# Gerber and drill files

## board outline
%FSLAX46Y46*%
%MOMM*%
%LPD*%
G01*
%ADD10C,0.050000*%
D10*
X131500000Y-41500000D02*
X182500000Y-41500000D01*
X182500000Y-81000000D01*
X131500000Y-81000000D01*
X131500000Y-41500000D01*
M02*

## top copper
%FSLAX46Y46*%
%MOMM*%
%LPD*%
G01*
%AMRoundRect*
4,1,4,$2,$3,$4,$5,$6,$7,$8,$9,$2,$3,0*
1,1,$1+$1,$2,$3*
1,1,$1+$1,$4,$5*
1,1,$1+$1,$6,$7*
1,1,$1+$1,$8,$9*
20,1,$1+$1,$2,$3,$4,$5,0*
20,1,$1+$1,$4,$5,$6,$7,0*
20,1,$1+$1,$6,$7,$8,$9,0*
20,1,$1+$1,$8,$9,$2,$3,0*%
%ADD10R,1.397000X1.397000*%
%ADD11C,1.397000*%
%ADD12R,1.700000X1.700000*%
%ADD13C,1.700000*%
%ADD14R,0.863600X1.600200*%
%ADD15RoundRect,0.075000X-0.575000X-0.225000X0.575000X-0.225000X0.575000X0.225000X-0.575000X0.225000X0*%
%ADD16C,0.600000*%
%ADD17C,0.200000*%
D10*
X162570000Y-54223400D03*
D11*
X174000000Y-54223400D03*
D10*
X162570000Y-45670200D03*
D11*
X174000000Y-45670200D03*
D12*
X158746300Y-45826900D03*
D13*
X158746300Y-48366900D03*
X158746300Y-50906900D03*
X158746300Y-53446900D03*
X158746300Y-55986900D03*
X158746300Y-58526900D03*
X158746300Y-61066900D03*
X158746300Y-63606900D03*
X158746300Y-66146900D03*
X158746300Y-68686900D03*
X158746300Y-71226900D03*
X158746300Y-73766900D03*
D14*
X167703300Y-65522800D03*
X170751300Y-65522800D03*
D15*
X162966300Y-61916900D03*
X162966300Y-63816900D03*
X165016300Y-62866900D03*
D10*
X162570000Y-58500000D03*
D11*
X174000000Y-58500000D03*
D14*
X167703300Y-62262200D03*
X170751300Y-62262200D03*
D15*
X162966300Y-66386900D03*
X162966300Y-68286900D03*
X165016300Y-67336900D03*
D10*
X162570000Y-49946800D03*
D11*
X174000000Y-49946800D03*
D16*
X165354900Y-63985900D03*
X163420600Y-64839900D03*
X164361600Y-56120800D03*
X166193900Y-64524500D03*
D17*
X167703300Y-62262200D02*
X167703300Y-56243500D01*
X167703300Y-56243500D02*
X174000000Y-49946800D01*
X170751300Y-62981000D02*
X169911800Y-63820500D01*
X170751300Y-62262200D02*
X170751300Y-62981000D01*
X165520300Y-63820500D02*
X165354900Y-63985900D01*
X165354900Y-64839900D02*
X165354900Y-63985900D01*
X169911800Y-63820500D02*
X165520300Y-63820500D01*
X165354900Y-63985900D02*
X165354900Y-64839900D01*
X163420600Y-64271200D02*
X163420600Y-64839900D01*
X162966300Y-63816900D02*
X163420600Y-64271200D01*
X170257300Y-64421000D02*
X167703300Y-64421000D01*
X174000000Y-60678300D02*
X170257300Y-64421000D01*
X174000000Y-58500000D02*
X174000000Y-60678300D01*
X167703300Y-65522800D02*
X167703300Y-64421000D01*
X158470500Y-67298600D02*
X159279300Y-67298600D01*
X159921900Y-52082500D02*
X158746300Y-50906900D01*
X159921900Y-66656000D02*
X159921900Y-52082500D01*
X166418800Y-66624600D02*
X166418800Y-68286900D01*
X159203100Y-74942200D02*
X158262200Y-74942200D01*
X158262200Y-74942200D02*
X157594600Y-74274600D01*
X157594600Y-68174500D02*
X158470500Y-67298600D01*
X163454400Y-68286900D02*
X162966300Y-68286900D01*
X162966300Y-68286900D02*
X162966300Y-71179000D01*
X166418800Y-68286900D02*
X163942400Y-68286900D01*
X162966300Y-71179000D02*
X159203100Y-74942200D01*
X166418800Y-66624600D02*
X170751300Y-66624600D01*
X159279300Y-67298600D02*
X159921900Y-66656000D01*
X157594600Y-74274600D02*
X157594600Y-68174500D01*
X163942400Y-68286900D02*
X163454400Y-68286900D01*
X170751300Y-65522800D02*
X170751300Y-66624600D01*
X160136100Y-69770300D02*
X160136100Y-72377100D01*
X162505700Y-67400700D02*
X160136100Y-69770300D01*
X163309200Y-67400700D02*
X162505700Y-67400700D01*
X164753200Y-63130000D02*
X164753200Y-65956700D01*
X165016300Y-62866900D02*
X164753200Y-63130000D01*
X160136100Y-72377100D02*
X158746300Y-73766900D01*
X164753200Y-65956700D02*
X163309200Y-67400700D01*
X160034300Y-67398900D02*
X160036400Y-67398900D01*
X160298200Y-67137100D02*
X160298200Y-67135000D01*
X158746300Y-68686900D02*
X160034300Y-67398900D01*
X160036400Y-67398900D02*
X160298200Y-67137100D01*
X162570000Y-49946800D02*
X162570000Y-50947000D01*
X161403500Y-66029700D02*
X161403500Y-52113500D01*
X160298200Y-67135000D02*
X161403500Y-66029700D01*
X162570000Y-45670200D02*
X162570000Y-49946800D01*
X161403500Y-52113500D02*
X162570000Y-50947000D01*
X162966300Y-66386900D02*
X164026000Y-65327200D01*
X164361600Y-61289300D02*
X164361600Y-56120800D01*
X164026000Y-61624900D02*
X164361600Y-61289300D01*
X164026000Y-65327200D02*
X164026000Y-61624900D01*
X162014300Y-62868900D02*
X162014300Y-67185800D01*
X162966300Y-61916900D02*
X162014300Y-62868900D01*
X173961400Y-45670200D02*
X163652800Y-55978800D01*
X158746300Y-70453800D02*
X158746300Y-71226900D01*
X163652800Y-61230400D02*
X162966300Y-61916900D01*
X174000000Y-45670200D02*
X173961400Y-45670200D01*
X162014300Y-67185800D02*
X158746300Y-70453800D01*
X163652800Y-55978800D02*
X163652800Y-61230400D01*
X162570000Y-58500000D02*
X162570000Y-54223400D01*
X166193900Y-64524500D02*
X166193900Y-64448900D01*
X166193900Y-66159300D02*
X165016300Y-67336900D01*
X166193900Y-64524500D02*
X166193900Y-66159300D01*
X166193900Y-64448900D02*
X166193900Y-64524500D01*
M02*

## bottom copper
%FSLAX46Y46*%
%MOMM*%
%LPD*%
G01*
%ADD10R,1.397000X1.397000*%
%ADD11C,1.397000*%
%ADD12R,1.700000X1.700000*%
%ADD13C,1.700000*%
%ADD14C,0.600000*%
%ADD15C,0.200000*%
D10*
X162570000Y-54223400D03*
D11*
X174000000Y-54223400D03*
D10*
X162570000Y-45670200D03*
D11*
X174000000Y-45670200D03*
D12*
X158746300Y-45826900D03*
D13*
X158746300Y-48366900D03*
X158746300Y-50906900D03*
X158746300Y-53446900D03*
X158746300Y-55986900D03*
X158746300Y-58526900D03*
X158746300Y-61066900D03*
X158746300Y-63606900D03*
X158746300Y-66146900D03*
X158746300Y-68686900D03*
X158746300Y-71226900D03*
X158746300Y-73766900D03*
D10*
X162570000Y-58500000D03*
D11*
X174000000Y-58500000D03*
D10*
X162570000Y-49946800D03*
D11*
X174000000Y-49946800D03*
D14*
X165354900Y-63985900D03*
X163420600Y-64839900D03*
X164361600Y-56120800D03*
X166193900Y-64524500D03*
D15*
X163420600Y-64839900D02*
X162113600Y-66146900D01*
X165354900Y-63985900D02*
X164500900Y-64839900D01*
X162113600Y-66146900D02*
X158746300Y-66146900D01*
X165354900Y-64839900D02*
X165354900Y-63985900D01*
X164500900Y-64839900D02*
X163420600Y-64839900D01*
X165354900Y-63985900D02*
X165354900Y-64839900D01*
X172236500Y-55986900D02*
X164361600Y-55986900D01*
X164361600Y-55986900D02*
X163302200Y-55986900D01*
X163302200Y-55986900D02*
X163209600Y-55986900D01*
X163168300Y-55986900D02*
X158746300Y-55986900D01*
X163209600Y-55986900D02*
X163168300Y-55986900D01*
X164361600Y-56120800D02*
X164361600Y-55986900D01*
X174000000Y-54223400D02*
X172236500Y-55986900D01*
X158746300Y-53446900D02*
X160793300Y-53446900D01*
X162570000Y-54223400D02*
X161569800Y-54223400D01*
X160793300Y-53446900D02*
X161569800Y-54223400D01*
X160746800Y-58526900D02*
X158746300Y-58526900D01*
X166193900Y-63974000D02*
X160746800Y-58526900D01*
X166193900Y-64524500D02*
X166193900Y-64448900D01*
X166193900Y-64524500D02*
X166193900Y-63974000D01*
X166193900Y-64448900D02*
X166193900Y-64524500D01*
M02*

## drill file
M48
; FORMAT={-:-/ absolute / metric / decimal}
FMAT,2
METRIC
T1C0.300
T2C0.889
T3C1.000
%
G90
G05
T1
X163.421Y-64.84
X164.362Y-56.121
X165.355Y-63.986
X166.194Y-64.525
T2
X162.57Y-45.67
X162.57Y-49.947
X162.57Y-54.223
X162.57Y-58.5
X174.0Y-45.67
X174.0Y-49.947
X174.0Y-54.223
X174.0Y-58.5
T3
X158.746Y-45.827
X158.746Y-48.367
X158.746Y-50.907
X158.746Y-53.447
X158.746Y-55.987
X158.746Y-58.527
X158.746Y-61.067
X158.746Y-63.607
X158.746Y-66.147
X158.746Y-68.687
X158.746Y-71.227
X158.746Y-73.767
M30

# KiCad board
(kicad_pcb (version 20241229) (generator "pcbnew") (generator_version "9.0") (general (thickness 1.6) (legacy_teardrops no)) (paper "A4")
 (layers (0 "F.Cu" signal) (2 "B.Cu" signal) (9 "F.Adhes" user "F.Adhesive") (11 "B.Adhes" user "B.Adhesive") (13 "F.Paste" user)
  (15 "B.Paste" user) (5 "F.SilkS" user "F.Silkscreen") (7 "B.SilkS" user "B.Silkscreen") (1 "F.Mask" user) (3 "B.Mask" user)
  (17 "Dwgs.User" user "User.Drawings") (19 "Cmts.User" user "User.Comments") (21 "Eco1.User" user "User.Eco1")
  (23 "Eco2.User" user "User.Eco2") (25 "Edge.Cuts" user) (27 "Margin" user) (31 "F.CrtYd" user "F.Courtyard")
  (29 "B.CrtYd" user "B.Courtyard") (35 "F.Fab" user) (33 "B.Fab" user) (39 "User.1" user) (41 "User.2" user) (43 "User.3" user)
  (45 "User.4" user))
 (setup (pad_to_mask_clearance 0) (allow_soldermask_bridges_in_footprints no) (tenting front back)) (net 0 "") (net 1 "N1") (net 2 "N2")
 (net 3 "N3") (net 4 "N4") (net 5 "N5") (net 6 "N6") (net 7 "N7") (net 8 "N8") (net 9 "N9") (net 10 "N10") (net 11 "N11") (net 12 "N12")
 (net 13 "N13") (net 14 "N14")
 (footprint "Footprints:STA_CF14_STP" (layer "F.Cu") (at 162.57 54.2234)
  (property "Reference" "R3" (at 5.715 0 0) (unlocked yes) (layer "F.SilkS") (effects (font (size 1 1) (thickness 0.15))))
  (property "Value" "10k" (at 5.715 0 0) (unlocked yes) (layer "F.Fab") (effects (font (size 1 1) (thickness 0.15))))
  (pad "1" thru_hole rect (at 0 0) (size 1.397 1.397) (drill 0.889) (layers "*.Cu" "*.Mask") (remove_unused_layers no) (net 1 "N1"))
  (pad "2" thru_hole circle (at 11.43 0) (size 1.397 1.397) (drill 0.889) (layers "*.Cu" "*.Mask") (remove_unused_layers no) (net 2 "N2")))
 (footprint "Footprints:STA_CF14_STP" (layer "F.Cu") (at 162.57 45.6702)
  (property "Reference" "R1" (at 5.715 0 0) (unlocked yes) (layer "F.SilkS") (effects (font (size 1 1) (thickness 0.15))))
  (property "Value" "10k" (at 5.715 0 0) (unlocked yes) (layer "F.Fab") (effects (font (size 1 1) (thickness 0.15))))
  (pad "1" thru_hole rect (at 0 0) (size 1.397 1.397) (drill 0.889) (layers "*.Cu" "*.Mask") (remove_unused_layers no) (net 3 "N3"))
  (pad "2" thru_hole circle (at 11.43 0) (size 1.397 1.397) (drill 0.889) (layers "*.Cu" "*.Mask") (remove_unused_layers no) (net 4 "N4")))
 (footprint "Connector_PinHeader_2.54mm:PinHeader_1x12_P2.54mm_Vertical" (layer "F.Cu") (at 158.7463 45.8269)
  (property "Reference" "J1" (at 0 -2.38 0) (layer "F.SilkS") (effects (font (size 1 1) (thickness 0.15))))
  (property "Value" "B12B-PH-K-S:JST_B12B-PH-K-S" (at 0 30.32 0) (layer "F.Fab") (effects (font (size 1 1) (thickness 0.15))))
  (pad "1" thru_hole rect (at 0 0) (size 1.7 1.7) (drill 1) (layers "*.Cu" "*.Mask") (remove_unused_layers no) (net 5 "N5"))
  (pad "2" thru_hole circle (at 0 2.54) (size 1.7 1.7) (drill 1) (layers "*.Cu" "*.Mask") (remove_unused_layers no) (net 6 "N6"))
  (pad "3" thru_hole circle (at 0 5.08) (size 1.7 1.7) (drill 1) (layers "*.Cu" "*.Mask") (remove_unused_layers no) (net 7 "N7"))
  (pad "4" thru_hole circle (at 0 7.62) (size 1.7 1.7) (drill 1) (layers "*.Cu" "*.Mask") (remove_unused_layers no) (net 1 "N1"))
  (pad "5" thru_hole circle (at 0 10.16) (size 1.7 1.7) (drill 1) (layers "*.Cu" "*.Mask") (remove_unused_layers no) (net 2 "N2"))
  (pad "6" thru_hole circle (at 0 12.7) (size 1.7 1.7) (drill 1) (layers "*.Cu" "*.Mask") (remove_unused_layers no) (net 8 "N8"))
  (pad "7" thru_hole circle (at 0 15.24) (size 1.7 1.7) (drill 1) (layers "*.Cu" "*.Mask") (remove_unused_layers no) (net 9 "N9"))
  (pad "8" thru_hole circle (at 0 17.78) (size 1.7 1.7) (drill 1) (layers "*.Cu" "*.Mask") (remove_unused_layers no) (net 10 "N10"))
  (pad "9" thru_hole circle (at 0 20.32) (size 1.7 1.7) (drill 1) (layers "*.Cu" "*.Mask") (remove_unused_layers no) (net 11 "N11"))
  (pad "10" thru_hole circle (at 0 22.86) (size 1.7 1.7) (drill 1) (layers "*.Cu" "*.Mask") (remove_unused_layers no) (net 3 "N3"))
  (pad "11" thru_hole circle (at 0 25.4) (size 1.7 1.7) (drill 1) (layers "*.Cu" "*.Mask") (remove_unused_layers no) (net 4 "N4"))
  (pad "12" thru_hole circle (at 0 27.94) (size 1.7 1.7) (drill 1) (layers "*.Cu" "*.Mask") (remove_unused_layers no) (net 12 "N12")))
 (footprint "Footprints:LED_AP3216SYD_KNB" (layer "F.Cu") (at 169.2273 65.5228)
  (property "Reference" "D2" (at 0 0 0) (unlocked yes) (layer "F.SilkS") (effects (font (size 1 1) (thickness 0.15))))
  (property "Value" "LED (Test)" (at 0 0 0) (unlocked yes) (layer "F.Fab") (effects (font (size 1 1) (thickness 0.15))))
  (pad "1" smd rect (at -1.524 0) (size 0.8636 1.6002) (layers "F.Cu" "F.Mask" "F.Paste") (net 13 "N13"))
  (pad "2" smd rect (at 1.524 0) (size 0.8636 1.6002) (layers "F.Cu" "F.Mask" "F.Paste") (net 7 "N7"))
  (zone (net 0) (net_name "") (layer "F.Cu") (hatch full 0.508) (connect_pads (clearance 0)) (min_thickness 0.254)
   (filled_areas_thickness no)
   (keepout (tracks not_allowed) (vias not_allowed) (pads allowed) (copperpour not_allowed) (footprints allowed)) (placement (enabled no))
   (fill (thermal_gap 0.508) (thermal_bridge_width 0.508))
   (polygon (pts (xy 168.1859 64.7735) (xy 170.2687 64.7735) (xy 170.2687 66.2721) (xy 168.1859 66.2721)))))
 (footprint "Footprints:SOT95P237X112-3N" (layer "F.Cu") (at 163.9913 62.8669)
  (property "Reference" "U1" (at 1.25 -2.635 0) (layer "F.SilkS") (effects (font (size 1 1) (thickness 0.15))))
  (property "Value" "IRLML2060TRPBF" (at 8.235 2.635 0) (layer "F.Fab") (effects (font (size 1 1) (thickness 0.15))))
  (pad "1" smd roundrect (at -1.025 -0.95) (size 1.3 0.6) (layers "F.Cu" "F.Mask" "F.Paste") (roundrect_rratio 0.125) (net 4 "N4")
   (solder_mask_margin 0.102))
  (pad "2" smd roundrect (at -1.025 0.95) (size 1.3 0.6) (layers "F.Cu" "F.Mask" "F.Paste") (roundrect_rratio 0.125) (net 11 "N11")
   (solder_mask_margin 0.102))
  (pad "3" smd roundrect (at 1.025 0) (size 1.3 0.6) (layers "F.Cu" "F.Mask" "F.Paste") (roundrect_rratio 0.125) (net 12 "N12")
   (solder_mask_margin 0.102)))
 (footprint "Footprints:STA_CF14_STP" (layer "F.Cu") (at 162.57 58.5)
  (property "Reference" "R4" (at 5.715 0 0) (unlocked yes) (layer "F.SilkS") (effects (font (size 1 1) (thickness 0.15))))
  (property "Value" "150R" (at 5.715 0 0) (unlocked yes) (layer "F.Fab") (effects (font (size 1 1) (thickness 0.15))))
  (pad "1" thru_hole rect (at 0 0) (size 1.397 1.397) (drill 0.889) (layers "*.Cu" "*.Mask") (remove_unused_layers no) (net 1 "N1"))
  (pad "2" thru_hole circle (at 11.43 0) (size 1.397 1.397) (drill 0.889) (layers "*.Cu" "*.Mask") (remove_unused_layers no) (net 13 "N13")))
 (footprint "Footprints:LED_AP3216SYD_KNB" (layer "F.Cu") (at 169.2273 62.2622)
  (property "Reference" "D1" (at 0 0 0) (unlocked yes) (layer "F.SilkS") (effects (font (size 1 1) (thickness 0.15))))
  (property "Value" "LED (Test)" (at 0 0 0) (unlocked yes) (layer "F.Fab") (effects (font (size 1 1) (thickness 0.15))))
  (pad "1" smd rect (at -1.524 0) (size 0.8636 1.6002) (layers "F.Cu" "F.Mask" "F.Paste") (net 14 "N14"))
  (pad "2" smd rect (at 1.524 0) (size 0.8636 1.6002) (layers "F.Cu" "F.Mask" "F.Paste") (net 11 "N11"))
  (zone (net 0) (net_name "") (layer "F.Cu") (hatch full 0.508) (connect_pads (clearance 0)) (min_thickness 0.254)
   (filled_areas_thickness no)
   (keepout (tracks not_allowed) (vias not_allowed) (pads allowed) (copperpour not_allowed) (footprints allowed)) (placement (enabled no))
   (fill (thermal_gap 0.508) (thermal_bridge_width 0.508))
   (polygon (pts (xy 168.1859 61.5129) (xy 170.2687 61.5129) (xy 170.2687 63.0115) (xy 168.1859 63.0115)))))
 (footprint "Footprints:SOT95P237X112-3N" (layer "F.Cu") (at 163.9913 67.3369)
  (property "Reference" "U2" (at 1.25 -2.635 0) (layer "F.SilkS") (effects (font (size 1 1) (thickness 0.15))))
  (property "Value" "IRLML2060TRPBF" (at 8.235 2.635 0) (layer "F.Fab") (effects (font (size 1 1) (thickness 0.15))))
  (pad "1" smd roundrect (at -1.025 -0.95) (size 1.3 0.6) (layers "F.Cu" "F.Mask" "F.Paste") (roundrect_rratio 0.125) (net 2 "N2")
   (solder_mask_margin 0.102))
  (pad "2" smd roundrect (at -1.025 0.95) (size 1.3 0.6) (layers "F.Cu" "F.Mask" "F.Paste") (roundrect_rratio 0.125) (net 7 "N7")
   (solder_mask_margin 0.102))
  (pad "3" smd roundrect (at 1.025 0) (size 1.3 0.6) (layers "F.Cu" "F.Mask" "F.Paste") (roundrect_rratio 0.125) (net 8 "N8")
   (solder_mask_margin 0.102)))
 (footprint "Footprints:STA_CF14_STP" (layer "F.Cu") (at 162.57 49.9468)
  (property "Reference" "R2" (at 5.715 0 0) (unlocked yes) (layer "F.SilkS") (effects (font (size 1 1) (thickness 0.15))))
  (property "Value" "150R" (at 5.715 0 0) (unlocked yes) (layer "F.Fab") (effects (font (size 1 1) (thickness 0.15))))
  (pad "1" thru_hole rect (at 0 0) (size 1.397 1.397) (drill 0.889) (layers "*.Cu" "*.Mask") (remove_unused_layers no) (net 3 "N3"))
  (pad "2" thru_hole circle (at 11.43 0) (size 1.397 1.397) (drill 0.889) (layers "*.Cu" "*.Mask") (remove_unused_layers no) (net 14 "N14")))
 (gr_rect (start 131.5 41.5) (end 182.5 81) (stroke (width 0.05) (type solid)) (fill no) (layer "Edge.Cuts"))
 (segment (start 167.7033 62.2622) (end 167.7033 56.2435) (width 0.2) (layer "F.Cu") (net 14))
 (segment (start 167.7033 56.2435) (end 174 49.9468) (width 0.2) (layer "F.Cu") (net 14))
 (segment (start 170.7513 62.981) (end 169.9118 63.8205) (width 0.2) (layer "F.Cu") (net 11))
 (segment (start 170.7513 62.2622) (end 170.7513 62.981) (width 0.2) (layer "F.Cu") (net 11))
 (segment (start 165.5203 63.8205) (end 165.3549 63.9859) (width 0.2) (layer "F.Cu") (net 11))
 (segment (start 165.3549 64.8399) (end 165.3549 63.9859) (width 0.2) (layer "F.Cu") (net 11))
 (segment (start 169.9118 63.8205) (end 165.5203 63.8205) (width 0.2) (layer "F.Cu") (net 11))
 (segment (start 165.3549 63.9859) (end 165.3549 64.8399) (width 0.2) (layer "F.Cu") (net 11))
 (segment (start 163.4206 64.2712) (end 163.4206 64.8399) (width 0.2) (layer "F.Cu") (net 11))
 (segment (start 162.9663 63.8169) (end 163.4206 64.2712) (width 0.2) (layer "F.Cu") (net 11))
 (via (at 165.3549 63.9859) (size 0.6) (drill 0.3) (layers "F.Cu" "B.Cu") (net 11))
 (via (at 163.4206 64.8399) (size 0.6) (drill 0.3) (layers "F.Cu" "B.Cu") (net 11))
 (segment (start 163.4206 64.8399) (end 162.1136 66.1469) (width 0.2) (layer "B.Cu") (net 11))
 (segment (start 165.3549 63.9859) (end 164.5009 64.8399) (width 0.2) (layer "B.Cu") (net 11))
 (segment (start 162.1136 66.1469) (end 158.7463 66.1469) (width 0.2) (layer "B.Cu") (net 11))
 (segment (start 165.3549 64.8399) (end 165.3549 63.9859) (width 0.2) (layer "B.Cu") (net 11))
 (segment (start 164.5009 64.8399) (end 163.4206 64.8399) (width 0.2) (layer "B.Cu") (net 11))
 (segment (start 165.3549 63.9859) (end 165.3549 64.8399) (width 0.2) (layer "B.Cu") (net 11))
 (segment (start 170.2573 64.421) (end 167.7033 64.421) (width 0.2) (layer "F.Cu") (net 13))
 (segment (start 174 60.6783) (end 170.2573 64.421) (width 0.2) (layer "F.Cu") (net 13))
 (segment (start 174 58.5) (end 174 60.6783) (width 0.2) (layer "F.Cu") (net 13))
 (segment (start 167.7033 65.5228) (end 167.7033 64.421) (width 0.2) (layer "F.Cu") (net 13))
 (segment (start 158.4705 67.2986) (end 159.2793 67.2986) (width 0.2) (layer "F.Cu") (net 7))
 (segment (start 159.9219 52.0825) (end 158.7463 50.9069) (width 0.2) (layer "F.Cu") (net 7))
 (segment (start 159.9219 66.656) (end 159.9219 52.0825) (width 0.2) (layer "F.Cu") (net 7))
 (segment (start 166.4188 66.6246) (end 166.4188 68.2869) (width 0.2) (layer "F.Cu") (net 7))
 (segment (start 159.2031 74.9422) (end 158.2622 74.9422) (width 0.2) (layer "F.Cu") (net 7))
 (segment (start 158.2622 74.9422) (end 157.5946 74.2746) (width 0.2) (layer "F.Cu") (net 7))
 (segment (start 157.5946 68.1745) (end 158.4705 67.2986) (width 0.2) (layer "F.Cu") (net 7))
 (segment (start 163.4544 68.2869) (end 162.9663 68.2869) (width 0.2) (layer "F.Cu") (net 7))
 (segment (start 162.9663 68.2869) (end 162.9663 71.179) (width 0.2) (layer "F.Cu") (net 7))
 (segment (start 166.4188 68.2869) (end 163.9424 68.2869) (width 0.2) (layer "F.Cu") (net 7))
 (segment (start 162.9663 71.179) (end 159.2031 74.9422) (width 0.2) (layer "F.Cu") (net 7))
 (segment (start 166.4188 66.6246) (end 170.7513 66.6246) (width 0.2) (layer "F.Cu") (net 7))
 (segment (start 159.2793 67.2986) (end 159.9219 66.656) (width 0.2) (layer "F.Cu") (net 7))
 (segment (start 157.5946 74.2746) (end 157.5946 68.1745) (width 0.2) (layer "F.Cu") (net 7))
 (segment (start 163.9424 68.2869) (end 163.4544 68.2869) (width 0.2) (layer "F.Cu") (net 7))
 (segment (start 170.7513 65.5228) (end 170.7513 66.6246) (width 0.2) (layer "F.Cu") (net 7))
 (segment (start 160.1361 69.7703) (end 160.1361 72.3771) (width 0.2) (layer "F.Cu") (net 12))
 (segment (start 162.5057 67.4007) (end 160.1361 69.7703) (width 0.2) (layer "F.Cu") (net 12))
 (segment (start 163.3092 67.4007) (end 162.5057 67.4007) (width 0.2) (layer "F.Cu") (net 12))
 (segment (start 164.7532 63.13) (end 164.7532 65.9567) (width 0.2) (layer "F.Cu") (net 12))
 (segment (start 165.0163 62.8669) (end 164.7532 63.13) (width 0.2) (layer "F.Cu") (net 12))
 (segment (start 160.1361 72.3771) (end 158.7463 73.7669) (width 0.2) (layer "F.Cu") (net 12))
 (segment (start 164.7532 65.9567) (end 163.3092 67.4007) (width 0.2) (layer "F.Cu") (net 12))
 (segment (start 160.0343 67.3989) (end 160.0364 67.3989) (width 0.2) (layer "F.Cu") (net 3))
 (segment (start 160.2982 67.1371) (end 160.2982 67.135) (width 0.2) (layer "F.Cu") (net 3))
 (segment (start 158.7463 68.6869) (end 160.0343 67.3989) (width 0.2) (layer "F.Cu") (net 3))
 (segment (start 160.0364 67.3989) (end 160.2982 67.1371) (width 0.2) (layer "F.Cu") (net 3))
 (segment (start 162.57 49.9468) (end 162.57 50.947) (width 0.2) (layer "F.Cu") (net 3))
 (segment (start 161.4035 66.0297) (end 161.4035 52.1135) (width 0.2) (layer "F.Cu") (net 3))
 (segment (start 160.2982 67.135) (end 161.4035 66.0297) (width 0.2) (layer "F.Cu") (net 3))
 (segment (start 162.57 45.6702) (end 162.57 49.9468) (width 0.2) (layer "F.Cu") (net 3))
 (segment (start 161.4035 52.1135) (end 162.57 50.947) (width 0.2) (layer "F.Cu") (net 3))
 (segment (start 162.9663 66.3869) (end 164.026 65.3272) (width 0.2) (layer "F.Cu") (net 2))
 (segment (start 164.3616 61.2893) (end 164.3616 56.1208) (width 0.2) (layer "F.Cu") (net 2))
 (segment (start 164.026 61.6249) (end 164.3616 61.2893) (width 0.2) (layer "F.Cu") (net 2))
 (segment (start 164.026 65.3272) (end 164.026 61.6249) (width 0.2) (layer "F.Cu") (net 2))
 (via (at 164.3616 56.1208) (size 0.6) (drill 0.3) (layers "F.Cu" "B.Cu") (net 2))
 (segment (start 172.2365 55.9869) (end 164.3616 55.9869) (width 0.2) (layer "B.Cu") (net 2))
 (segment (start 164.3616 55.9869) (end 163.3022 55.9869) (width 0.2) (layer "B.Cu") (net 2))
 (segment (start 163.3022 55.9869) (end 163.2096 55.9869) (width 0.2) (layer "B.Cu") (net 2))
 (segment (start 163.1683 55.9869) (end 158.7463 55.9869) (width 0.2) (layer "B.Cu") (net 2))
 (segment (start 163.2096 55.9869) (end 163.1683 55.9869) (width 0.2) (layer "B.Cu") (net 2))
 (segment (start 164.3616 56.1208) (end 164.3616 55.9869) (width 0.2) (layer "B.Cu") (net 2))
 (segment (start 174 54.2234) (end 172.2365 55.9869) (width 0.2) (layer "B.Cu") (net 2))
 (segment (start 162.0143 62.8689) (end 162.0143 67.1858) (width 0.2) (layer "F.Cu") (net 4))
 (segment (start 162.9663 61.9169) (end 162.0143 62.8689) (width 0.2) (layer "F.Cu") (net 4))
 (segment (start 173.9614 45.6702) (end 163.6528 55.9788) (width 0.2) (layer "F.Cu") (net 4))
 (segment (start 158.7463 70.4538) (end 158.7463 71.2269) (width 0.2) (layer "F.Cu") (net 4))
 (segment (start 163.6528 61.2304) (end 162.9663 61.9169) (width 0.2) (layer "F.Cu") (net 4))
 (segment (start 174 45.6702) (end 173.9614 45.6702) (width 0.2) (layer "F.Cu") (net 4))
 (segment (start 162.0143 67.1858) (end 158.7463 70.4538) (width 0.2) (layer "F.Cu") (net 4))
 (segment (start 163.6528 55.9788) (end 163.6528 61.2304) (width 0.2) (layer "F.Cu") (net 4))
 (segment (start 162.57 58.5) (end 162.57 54.2234) (width 0.2) (layer "F.Cu") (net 1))
 (segment (start 158.7463 53.4469) (end 160.7933 53.4469) (width 0.2) (layer "B.Cu") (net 1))
 (segment (start 162.57 54.2234) (end 161.5698 54.2234) (width 0.2) (layer "B.Cu") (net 1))
 (segment (start 160.7933 53.4469) (end 161.5698 54.2234) (width 0.2) (layer "B.Cu") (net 1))
 (segment (start 166.1939 64.5245) (end 166.1939 64.4489) (width 0.2) (layer "F.Cu") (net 8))
 (segment (start 166.1939 66.1593) (end 165.0163 67.3369) (width 0.2) (layer "F.Cu") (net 8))
 (segment (start 166.1939 64.5245) (end 166.1939 66.1593) (width 0.2) (layer "F.Cu") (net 8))
 (segment (start 166.1939 64.4489) (end 166.1939 64.5245) (width 0.2) (layer "F.Cu") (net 8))
 (via (at 166.1939 64.5245) (size 0.6) (drill 0.3) (layers "F.Cu" "B.Cu") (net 8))
 (segment (start 160.7468 58.5269) (end 158.7463 58.5269) (width 0.2) (layer "B.Cu") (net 8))
 (segment (start 166.1939 63.974) (end 160.7468 58.5269) (width 0.2) (layer "B.Cu") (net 8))
 (segment (start 166.1939 64.5245) (end 166.1939 64.4489) (width 0.2) (layer "B.Cu") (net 8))
 (segment (start 166.1939 64.5245) (end 166.1939 63.974) (width 0.2) (layer "B.Cu") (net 8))
 (segment (start 166.1939 64.4489) (end 166.1939 64.5245) (width 0.2) (layer "B.Cu") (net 8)))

